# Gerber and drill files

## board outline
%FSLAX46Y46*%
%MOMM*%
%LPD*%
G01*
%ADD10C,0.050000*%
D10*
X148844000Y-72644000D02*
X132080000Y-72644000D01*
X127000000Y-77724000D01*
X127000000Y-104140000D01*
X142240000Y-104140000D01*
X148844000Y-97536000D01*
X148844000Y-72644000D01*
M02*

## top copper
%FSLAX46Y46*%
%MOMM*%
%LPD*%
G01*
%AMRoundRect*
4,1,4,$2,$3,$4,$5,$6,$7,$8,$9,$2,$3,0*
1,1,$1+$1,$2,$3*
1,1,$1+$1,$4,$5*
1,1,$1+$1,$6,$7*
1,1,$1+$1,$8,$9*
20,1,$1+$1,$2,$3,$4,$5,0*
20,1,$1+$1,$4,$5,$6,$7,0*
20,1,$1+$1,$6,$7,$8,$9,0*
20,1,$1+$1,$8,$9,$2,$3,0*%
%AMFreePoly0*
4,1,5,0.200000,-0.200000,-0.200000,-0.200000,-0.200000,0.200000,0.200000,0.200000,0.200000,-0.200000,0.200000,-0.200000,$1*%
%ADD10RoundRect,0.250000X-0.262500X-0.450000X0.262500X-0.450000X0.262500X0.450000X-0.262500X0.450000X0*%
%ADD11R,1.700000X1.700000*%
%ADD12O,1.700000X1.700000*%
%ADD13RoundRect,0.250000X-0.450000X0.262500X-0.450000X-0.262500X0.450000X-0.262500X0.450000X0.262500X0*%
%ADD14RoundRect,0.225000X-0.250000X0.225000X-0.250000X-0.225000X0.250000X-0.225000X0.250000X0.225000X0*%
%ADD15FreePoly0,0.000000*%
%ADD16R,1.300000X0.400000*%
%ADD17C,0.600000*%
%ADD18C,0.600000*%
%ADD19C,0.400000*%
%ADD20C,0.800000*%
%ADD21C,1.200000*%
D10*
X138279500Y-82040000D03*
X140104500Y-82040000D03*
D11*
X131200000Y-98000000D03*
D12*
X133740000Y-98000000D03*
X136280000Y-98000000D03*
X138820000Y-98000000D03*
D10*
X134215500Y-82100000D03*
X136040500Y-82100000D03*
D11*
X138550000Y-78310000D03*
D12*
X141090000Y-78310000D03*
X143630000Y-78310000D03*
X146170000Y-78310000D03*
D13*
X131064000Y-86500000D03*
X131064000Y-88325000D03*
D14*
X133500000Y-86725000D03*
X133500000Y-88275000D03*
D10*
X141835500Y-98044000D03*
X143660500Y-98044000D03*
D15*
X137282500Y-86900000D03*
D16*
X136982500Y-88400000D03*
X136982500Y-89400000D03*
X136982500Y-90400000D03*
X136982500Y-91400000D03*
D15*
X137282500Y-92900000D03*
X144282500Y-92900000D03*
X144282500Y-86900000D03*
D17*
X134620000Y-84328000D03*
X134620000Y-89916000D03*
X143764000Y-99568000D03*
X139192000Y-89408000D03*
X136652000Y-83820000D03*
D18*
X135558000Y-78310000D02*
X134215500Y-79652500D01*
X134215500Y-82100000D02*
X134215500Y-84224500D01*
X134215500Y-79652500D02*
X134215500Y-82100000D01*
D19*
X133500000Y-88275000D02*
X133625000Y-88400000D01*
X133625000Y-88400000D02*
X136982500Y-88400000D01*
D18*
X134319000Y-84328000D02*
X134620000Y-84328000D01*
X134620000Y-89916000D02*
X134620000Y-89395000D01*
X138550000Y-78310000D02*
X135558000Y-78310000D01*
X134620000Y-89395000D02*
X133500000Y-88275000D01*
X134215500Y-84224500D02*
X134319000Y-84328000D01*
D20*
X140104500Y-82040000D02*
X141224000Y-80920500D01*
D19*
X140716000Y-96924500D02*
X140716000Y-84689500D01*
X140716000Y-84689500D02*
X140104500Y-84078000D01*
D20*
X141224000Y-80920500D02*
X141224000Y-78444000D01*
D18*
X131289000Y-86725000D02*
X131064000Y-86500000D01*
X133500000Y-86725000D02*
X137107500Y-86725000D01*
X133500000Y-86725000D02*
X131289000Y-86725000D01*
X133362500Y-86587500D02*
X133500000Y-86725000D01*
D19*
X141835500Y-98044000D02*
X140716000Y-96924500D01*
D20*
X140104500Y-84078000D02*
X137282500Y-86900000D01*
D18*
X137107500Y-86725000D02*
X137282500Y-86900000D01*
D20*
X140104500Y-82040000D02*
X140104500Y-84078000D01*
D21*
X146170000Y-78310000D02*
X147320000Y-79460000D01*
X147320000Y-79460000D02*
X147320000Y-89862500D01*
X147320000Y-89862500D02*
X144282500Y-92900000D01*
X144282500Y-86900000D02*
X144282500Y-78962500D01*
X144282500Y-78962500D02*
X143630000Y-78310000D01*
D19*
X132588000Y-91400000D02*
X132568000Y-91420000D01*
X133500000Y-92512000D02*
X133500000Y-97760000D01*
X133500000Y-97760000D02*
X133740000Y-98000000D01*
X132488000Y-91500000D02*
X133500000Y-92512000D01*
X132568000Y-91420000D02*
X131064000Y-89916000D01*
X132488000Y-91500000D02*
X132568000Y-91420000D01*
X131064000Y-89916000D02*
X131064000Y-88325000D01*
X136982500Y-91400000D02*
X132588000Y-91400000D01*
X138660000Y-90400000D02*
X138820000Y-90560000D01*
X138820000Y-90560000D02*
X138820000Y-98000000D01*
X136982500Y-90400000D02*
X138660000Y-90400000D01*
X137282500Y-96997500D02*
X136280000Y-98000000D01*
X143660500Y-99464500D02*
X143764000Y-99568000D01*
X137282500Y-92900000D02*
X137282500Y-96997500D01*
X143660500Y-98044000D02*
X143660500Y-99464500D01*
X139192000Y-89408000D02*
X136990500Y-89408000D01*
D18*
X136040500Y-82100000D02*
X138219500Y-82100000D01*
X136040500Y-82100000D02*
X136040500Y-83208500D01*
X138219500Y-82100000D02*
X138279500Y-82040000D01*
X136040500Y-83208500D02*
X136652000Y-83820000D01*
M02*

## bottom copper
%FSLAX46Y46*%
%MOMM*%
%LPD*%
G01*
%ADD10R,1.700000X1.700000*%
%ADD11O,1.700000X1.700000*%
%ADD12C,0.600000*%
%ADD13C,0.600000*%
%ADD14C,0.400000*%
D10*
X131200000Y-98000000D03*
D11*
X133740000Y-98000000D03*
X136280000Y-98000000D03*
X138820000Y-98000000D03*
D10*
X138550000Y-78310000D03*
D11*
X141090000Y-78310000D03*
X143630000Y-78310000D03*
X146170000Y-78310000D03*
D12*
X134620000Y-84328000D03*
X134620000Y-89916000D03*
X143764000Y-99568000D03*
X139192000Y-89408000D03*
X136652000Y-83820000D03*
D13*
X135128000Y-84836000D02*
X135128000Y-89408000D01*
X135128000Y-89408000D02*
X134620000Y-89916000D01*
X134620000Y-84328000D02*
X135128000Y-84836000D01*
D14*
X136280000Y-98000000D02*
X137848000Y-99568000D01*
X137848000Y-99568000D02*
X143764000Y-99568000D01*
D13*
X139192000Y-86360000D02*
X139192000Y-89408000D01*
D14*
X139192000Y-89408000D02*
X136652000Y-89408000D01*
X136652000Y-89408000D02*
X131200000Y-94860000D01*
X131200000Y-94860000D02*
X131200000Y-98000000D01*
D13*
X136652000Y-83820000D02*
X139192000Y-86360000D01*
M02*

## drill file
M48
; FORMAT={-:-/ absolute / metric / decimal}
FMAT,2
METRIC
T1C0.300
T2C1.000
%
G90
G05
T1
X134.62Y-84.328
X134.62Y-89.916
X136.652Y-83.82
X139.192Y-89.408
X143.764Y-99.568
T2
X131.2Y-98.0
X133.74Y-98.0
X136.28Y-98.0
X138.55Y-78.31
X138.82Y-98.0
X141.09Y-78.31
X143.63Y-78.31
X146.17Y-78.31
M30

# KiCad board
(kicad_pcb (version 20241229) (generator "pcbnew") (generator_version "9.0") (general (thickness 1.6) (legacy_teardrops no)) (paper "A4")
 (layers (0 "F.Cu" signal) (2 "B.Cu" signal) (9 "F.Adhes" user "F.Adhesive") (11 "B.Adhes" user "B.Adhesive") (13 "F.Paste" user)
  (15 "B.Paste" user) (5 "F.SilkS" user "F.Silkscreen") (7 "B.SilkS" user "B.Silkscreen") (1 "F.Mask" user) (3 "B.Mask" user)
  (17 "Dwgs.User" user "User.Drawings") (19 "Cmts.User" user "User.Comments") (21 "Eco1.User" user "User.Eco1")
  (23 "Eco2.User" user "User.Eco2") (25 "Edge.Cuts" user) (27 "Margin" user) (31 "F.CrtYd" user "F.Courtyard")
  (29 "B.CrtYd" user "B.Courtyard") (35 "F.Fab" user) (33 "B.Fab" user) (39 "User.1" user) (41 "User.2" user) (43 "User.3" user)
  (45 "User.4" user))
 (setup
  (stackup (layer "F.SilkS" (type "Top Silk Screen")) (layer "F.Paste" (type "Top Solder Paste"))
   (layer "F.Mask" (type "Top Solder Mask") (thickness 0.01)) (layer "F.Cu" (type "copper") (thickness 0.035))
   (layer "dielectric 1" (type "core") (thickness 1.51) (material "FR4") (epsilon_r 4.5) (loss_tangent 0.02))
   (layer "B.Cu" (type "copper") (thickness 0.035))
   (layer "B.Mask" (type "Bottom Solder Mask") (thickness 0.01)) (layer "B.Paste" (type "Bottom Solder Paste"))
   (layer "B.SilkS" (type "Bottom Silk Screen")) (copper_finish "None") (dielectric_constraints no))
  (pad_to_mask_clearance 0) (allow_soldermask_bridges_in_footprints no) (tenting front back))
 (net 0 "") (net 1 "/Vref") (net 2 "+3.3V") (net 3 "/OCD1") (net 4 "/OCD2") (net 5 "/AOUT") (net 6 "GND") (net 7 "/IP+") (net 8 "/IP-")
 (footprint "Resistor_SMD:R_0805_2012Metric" (layer "F.Cu") (at 139.192 82.04)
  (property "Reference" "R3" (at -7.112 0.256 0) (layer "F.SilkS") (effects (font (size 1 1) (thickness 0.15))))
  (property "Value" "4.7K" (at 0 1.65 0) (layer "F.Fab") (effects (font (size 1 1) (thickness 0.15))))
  (pad "1" smd roundrect (at -0.9125 0) (size 1.025 1.4) (layers "F.Cu" "F.Mask" "F.Paste") (roundrect_rratio 0.243902) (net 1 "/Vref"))
  (pad "2" smd roundrect (at 0.9125 0) (size 1.025 1.4) (layers "F.Cu" "F.Mask" "F.Paste") (roundrect_rratio 0.243902) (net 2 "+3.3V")))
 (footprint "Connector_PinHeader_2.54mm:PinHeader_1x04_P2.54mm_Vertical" (layer "F.Cu") (at 131.2 98 90)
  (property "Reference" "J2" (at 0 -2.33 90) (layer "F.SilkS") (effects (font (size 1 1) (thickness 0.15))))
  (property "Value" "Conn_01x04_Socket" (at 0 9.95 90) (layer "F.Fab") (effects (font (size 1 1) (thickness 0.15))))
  (pad "1" thru_hole rect (at 0 0 90) (size 1.7 1.7) (drill 1) (layers "*.Cu" "*.Mask") (remove_unused_layers no) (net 1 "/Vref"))
  (pad "2" thru_hole oval (at 0 2.54 90) (size 1.7 1.7) (drill 1) (layers "*.Cu" "*.Mask") (remove_unused_layers no) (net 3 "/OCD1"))
  (pad "3" thru_hole oval (at 0 5.08 90) (size 1.7 1.7) (drill 1) (layers "*.Cu" "*.Mask") (remove_unused_layers no) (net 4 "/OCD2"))
  (pad "4" thru_hole oval (at 0 7.62 90) (size 1.7 1.7) (drill 1) (layers "*.Cu" "*.Mask") (remove_unused_layers no) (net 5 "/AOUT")))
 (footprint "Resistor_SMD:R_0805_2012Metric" (layer "F.Cu") (at 135.128 82.1)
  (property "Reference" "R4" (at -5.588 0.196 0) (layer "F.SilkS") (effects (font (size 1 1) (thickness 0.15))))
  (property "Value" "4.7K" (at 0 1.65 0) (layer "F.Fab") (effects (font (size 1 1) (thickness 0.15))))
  (pad "1" smd roundrect (at -0.9125 0) (size 1.025 1.4) (layers "F.Cu" "F.Mask" "F.Paste") (roundrect_rratio 0.243902) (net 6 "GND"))
  (pad "2" smd roundrect (at 0.9125 0) (size 1.025 1.4) (layers "F.Cu" "F.Mask" "F.Paste") (roundrect_rratio 0.243902) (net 1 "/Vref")))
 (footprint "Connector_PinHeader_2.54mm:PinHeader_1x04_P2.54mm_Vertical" (layer "F.Cu") (at 138.55 78.31 90)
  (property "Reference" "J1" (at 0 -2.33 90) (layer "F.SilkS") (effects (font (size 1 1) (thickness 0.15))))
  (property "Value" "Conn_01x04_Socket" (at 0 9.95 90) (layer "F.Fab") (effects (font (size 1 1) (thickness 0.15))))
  (pad "1" thru_hole rect (at 0 0 90) (size 1.7 1.7) (drill 1) (layers "*.Cu" "*.Mask") (remove_unused_layers no) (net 6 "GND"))
  (pad "2" thru_hole oval (at 0 2.54 90) (size 1.7 1.7) (drill 1) (layers "*.Cu" "*.Mask") (remove_unused_layers no) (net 2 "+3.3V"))
  (pad "3" thru_hole oval (at 0 5.08 90) (size 1.7 1.7) (drill 1) (layers "*.Cu" "*.Mask") (remove_unused_layers no) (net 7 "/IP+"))
  (pad "4" thru_hole oval (at 0 7.62 90) (size 1.7 1.7) (drill 1) (layers "*.Cu" "*.Mask") (remove_unused_layers no) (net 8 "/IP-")))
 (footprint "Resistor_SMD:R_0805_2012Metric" (layer "F.Cu") (at 131.064 87.4125 -90)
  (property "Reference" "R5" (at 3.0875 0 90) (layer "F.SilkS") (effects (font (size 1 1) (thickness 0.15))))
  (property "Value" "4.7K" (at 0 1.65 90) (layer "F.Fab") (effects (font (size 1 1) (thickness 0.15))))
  (pad "1" smd roundrect (at -0.9125 0 270) (size 1.025 1.4) (layers "F.Cu" "F.Mask" "F.Paste") (roundrect_rratio 0.243902) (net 2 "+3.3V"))
  (pad "2" smd roundrect (at 0.9125 0 270) (size 1.025 1.4) (layers "F.Cu" "F.Mask" "F.Paste") (roundrect_rratio 0.243902) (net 3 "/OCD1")))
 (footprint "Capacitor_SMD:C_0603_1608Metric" (layer "F.Cu") (at 133.5 87.5 -90)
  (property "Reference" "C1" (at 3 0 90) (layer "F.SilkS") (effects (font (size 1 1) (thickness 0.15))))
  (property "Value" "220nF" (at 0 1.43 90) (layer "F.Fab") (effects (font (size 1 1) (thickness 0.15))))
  (pad "1" smd roundrect (at -0.775 0 270) (size 0.9 0.95) (layers "F.Cu" "F.Mask" "F.Paste") (roundrect_rratio 0.25) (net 2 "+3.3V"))
  (pad "2" smd roundrect (at 0.775 0 270) (size 0.9 0.95) (layers "F.Cu" "F.Mask" "F.Paste") (roundrect_rratio 0.25) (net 6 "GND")))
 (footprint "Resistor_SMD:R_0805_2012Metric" (layer "F.Cu") (at 142.748 98.044)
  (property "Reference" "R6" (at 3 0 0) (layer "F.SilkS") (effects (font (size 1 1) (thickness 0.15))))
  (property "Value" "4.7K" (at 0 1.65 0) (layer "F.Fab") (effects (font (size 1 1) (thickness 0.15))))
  (pad "1" smd roundrect (at -0.9125 0) (size 1.025 1.4) (layers "F.Cu" "F.Mask" "F.Paste") (roundrect_rratio 0.243902) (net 2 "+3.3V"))
  (pad "2" smd roundrect (at 0.9125 0) (size 1.025 1.4) (layers "F.Cu" "F.Mask" "F.Paste") (roundrect_rratio 0.243902) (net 4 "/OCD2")))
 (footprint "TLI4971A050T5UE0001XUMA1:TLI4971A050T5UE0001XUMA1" (layer "F.Cu") (at 140.7825 89.9)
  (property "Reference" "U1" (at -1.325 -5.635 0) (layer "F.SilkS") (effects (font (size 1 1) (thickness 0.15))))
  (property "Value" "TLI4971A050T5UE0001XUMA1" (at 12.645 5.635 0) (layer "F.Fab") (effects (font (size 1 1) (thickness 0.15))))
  (pad "1" smd custom (at -3.5 -3) (size 0.4 0.4) (layers "F.Cu") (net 2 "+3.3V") (options (clearance outline) (anchor rect)) (primitives))
  (pad "2" smd rect (at -3.8 -1.5) (size 1.3 0.4) (layers "F.Cu" "F.Mask") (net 6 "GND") (solder_mask_margin 0.102))
  (pad "3" smd rect (at -3.8 -0.5) (size 1.3 0.4) (layers "F.Cu" "F.Mask") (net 1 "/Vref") (solder_mask_margin 0.102))
  (pad "4" smd rect (at -3.8 0.5) (size 1.3 0.4) (layers "F.Cu" "F.Mask") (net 5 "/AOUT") (solder_mask_margin 0.102))
  (pad "5" smd rect (at -3.8 1.5) (size 1.3 0.4) (layers "F.Cu" "F.Mask") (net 3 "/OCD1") (solder_mask_margin 0.102))
  (pad "6" smd custom (at -3.5 3) (size 0.4 0.4) (layers "F.Cu") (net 4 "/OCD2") (options (clearance outline) (anchor rect)) (primitives))
  (pad "7" smd custom (at 3.5 3) (size 0.4 0.4) (layers "F.Cu") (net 8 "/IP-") (options (clearance outline) (anchor rect)) (primitives))
  (pad "8" smd custom (at 3.5 -3) (size 0.4 0.4) (layers "F.Cu") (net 7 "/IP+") (options (clearance outline) (anchor rect)) (primitives)))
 (gr_poly
  (pts (xy 148.844 72.644) (xy 132.08 72.644) (xy 127 77.724) (xy 127 104.14) (xy 127 104.14) (xy 142.24 104.14) (xy 148.844 97.536))
  (stroke (width 0.05) (type solid)) (fill no) (layer "Edge.Cuts"))
 (segment (start 135.558 78.31) (end 134.2155 79.6525) (width 0.6) (layer "F.Cu") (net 6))
 (segment (start 134.2155 82.1) (end 134.2155 84.2245) (width 0.6) (layer "F.Cu") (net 6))
 (segment (start 134.2155 79.6525) (end 134.2155 82.1) (width 0.6) (layer "F.Cu") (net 6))
 (segment (start 133.5 88.275) (end 133.625 88.4) (width 0.4) (layer "F.Cu") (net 6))
 (segment (start 133.625 88.4) (end 136.9825 88.4) (width 0.4) (layer "F.Cu") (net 6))
 (segment (start 134.319 84.328) (end 134.62 84.328) (width 0.6) (layer "F.Cu") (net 6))
 (segment (start 134.62 89.916) (end 134.62 89.395) (width 0.6) (layer "F.Cu") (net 6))
 (segment (start 138.55 78.31) (end 135.558 78.31) (width 0.6) (layer "F.Cu") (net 6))
 (segment (start 134.62 89.395) (end 133.5 88.275) (width 0.6) (layer "F.Cu") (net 6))
 (segment (start 134.2155 84.2245) (end 134.319 84.328) (width 0.6) (layer "F.Cu") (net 6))
 (via (at 134.62 84.328) (size 0.6) (drill 0.3) (layers "F.Cu" "B.Cu") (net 6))
 (via (at 134.62 89.916) (size 0.6) (drill 0.3) (layers "F.Cu" "B.Cu") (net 6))
 (segment (start 135.128 84.836) (end 135.128 89.408) (width 0.6) (layer "B.Cu") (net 6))
 (segment (start 135.128 89.408) (end 134.62 89.916) (width 0.6) (layer "B.Cu") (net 6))
 (segment (start 134.62 84.328) (end 135.128 84.836) (width 0.6) (layer "B.Cu") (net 6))
 (segment (start 140.1045 82.04) (end 141.224 80.9205) (width 0.8) (layer "F.Cu") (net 2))
 (segment (start 140.716 96.9245) (end 140.716 84.6895) (width 0.4) (layer "F.Cu") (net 2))
 (segment (start 140.716 84.6895) (end 140.1045 84.078) (width 0.4) (layer "F.Cu") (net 2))
 (segment (start 141.224 80.9205) (end 141.224 78.444) (width 0.8) (layer "F.Cu") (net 2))
 (segment (start 131.289 86.725) (end 131.064 86.5) (width 0.6) (layer "F.Cu") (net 2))
 (segment (start 133.5 86.725) (end 137.1075 86.725) (width 0.6) (layer "F.Cu") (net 2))
 (segment (start 133.5 86.725) (end 131.289 86.725) (width 0.6) (layer "F.Cu") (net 2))
 (segment (start 133.3625 86.5875) (end 133.5 86.725) (width 0.6) (layer "F.Cu") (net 2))
 (segment (start 141.8355 98.044) (end 140.716 96.9245) (width 0.4) (layer "F.Cu") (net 2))
 (segment (start 140.1045 84.078) (end 137.2825 86.9) (width 0.8) (layer "F.Cu") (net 2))
 (segment (start 137.1075 86.725) (end 137.2825 86.9) (width 0.6) (layer "F.Cu") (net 2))
 (segment (start 140.1045 82.04) (end 140.1045 84.078) (width 0.8) (layer "F.Cu") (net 2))
 (segment (start 146.17 78.31) (end 147.32 79.46) (width 1.2) (layer "F.Cu") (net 8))
 (segment (start 147.32 79.46) (end 147.32 89.8625) (width 1.2) (layer "F.Cu") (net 8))
 (segment (start 147.32 89.8625) (end 144.2825 92.9) (width 1.2) (layer "F.Cu") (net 8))
 (segment (start 144.2825 86.9) (end 144.2825 78.9625) (width 1.2) (layer "F.Cu") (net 7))
 (segment (start 144.2825 78.9625) (end 143.63 78.31) (width 1.2) (layer "F.Cu") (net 7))
 (segment (start 132.588 91.4) (end 132.568 91.42) (width 0.4) (layer "F.Cu") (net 3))
 (segment (start 133.5 92.512) (end 133.5 97.76) (width 0.4) (layer "F.Cu") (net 3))
 (segment (start 133.5 97.76) (end 133.74 98) (width 0.4) (layer "F.Cu") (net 3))
 (segment (start 132.488 91.5) (end 133.5 92.512) (width 0.4) (layer "F.Cu") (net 3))
 (segment (start 132.568 91.42) (end 131.064 89.916) (width 0.4) (layer "F.Cu") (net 3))
 (segment (start 132.488 91.5) (end 132.568 91.42) (width 0.4) (layer "F.Cu") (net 3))
 (segment (start 131.064 89.916) (end 131.064 88.325) (width 0.4) (layer "F.Cu") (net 3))
 (segment (start 136.9825 91.4) (end 132.588 91.4) (width 0.4) (layer "F.Cu") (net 3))
 (segment (start 138.66 90.4) (end 138.82 90.56) (width 0.4) (layer "F.Cu") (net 5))
 (segment (start 138.82 90.56) (end 138.82 98) (width 0.4) (layer "F.Cu") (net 5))
 (segment (start 136.9825 90.4) (end 138.66 90.4) (width 0.4) (layer "F.Cu") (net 5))
 (segment (start 137.2825 96.9975) (end 136.28 98) (width 0.4) (layer "F.Cu") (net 4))
 (segment (start 143.6605 99.4645) (end 143.764 99.568) (width 0.4) (layer "F.Cu") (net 4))
 (segment (start 137.2825 92.9) (end 137.2825 96.9975) (width 0.4) (layer "F.Cu") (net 4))
 (segment (start 143.6605 98.044) (end 143.6605 99.4645) (width 0.4) (layer "F.Cu") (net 4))
 (via (at 143.764 99.568) (size 0.6) (drill 0.3) (layers "F.Cu" "B.Cu") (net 4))
 (segment (start 136.28 98) (end 137.848 99.568) (width 0.4) (layer "B.Cu") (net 4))
 (segment (start 137.848 99.568) (end 143.764 99.568) (width 0.4) (layer "B.Cu") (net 4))
 (segment (start 139.192 89.408) (end 136.9905 89.408) (width 0.4) (layer "F.Cu") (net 1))
 (segment (start 136.0405 82.1) (end 138.2195 82.1) (width 0.6) (layer "F.Cu") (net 1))
 (segment (start 136.0405 82.1) (end 136.0405 83.2085) (width 0.6) (layer "F.Cu") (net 1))
 (segment (start 138.2195 82.1) (end 138.2795 82.04) (width 0.6) (layer "F.Cu") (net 1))
 (segment (start 136.0405 83.2085) (end 136.652 83.82) (width 0.6) (layer "F.Cu") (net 1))
 (via (at 139.192 89.408) (size 0.6) (drill 0.3) (layers "F.Cu" "B.Cu") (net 1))
 (via (at 136.652 83.82) (size 0.6) (drill 0.3) (layers "F.Cu" "B.Cu") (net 1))
 (segment (start 139.192 86.36) (end 139.192 89.408) (width 0.6) (layer "B.Cu") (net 1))
 (segment (start 139.192 89.408) (end 136.652 89.408) (width 0.4) (layer "B.Cu") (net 1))
 (segment (start 136.652 89.408) (end 131.2 94.86) (width 0.4) (layer "B.Cu") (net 1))
 (segment (start 131.2 94.86) (end 131.2 98) (width 0.4) (layer "B.Cu") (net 1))
 (segment (start 136.652 83.82) (end 139.192 86.36) (width 0.6) (layer "B.Cu") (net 1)))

